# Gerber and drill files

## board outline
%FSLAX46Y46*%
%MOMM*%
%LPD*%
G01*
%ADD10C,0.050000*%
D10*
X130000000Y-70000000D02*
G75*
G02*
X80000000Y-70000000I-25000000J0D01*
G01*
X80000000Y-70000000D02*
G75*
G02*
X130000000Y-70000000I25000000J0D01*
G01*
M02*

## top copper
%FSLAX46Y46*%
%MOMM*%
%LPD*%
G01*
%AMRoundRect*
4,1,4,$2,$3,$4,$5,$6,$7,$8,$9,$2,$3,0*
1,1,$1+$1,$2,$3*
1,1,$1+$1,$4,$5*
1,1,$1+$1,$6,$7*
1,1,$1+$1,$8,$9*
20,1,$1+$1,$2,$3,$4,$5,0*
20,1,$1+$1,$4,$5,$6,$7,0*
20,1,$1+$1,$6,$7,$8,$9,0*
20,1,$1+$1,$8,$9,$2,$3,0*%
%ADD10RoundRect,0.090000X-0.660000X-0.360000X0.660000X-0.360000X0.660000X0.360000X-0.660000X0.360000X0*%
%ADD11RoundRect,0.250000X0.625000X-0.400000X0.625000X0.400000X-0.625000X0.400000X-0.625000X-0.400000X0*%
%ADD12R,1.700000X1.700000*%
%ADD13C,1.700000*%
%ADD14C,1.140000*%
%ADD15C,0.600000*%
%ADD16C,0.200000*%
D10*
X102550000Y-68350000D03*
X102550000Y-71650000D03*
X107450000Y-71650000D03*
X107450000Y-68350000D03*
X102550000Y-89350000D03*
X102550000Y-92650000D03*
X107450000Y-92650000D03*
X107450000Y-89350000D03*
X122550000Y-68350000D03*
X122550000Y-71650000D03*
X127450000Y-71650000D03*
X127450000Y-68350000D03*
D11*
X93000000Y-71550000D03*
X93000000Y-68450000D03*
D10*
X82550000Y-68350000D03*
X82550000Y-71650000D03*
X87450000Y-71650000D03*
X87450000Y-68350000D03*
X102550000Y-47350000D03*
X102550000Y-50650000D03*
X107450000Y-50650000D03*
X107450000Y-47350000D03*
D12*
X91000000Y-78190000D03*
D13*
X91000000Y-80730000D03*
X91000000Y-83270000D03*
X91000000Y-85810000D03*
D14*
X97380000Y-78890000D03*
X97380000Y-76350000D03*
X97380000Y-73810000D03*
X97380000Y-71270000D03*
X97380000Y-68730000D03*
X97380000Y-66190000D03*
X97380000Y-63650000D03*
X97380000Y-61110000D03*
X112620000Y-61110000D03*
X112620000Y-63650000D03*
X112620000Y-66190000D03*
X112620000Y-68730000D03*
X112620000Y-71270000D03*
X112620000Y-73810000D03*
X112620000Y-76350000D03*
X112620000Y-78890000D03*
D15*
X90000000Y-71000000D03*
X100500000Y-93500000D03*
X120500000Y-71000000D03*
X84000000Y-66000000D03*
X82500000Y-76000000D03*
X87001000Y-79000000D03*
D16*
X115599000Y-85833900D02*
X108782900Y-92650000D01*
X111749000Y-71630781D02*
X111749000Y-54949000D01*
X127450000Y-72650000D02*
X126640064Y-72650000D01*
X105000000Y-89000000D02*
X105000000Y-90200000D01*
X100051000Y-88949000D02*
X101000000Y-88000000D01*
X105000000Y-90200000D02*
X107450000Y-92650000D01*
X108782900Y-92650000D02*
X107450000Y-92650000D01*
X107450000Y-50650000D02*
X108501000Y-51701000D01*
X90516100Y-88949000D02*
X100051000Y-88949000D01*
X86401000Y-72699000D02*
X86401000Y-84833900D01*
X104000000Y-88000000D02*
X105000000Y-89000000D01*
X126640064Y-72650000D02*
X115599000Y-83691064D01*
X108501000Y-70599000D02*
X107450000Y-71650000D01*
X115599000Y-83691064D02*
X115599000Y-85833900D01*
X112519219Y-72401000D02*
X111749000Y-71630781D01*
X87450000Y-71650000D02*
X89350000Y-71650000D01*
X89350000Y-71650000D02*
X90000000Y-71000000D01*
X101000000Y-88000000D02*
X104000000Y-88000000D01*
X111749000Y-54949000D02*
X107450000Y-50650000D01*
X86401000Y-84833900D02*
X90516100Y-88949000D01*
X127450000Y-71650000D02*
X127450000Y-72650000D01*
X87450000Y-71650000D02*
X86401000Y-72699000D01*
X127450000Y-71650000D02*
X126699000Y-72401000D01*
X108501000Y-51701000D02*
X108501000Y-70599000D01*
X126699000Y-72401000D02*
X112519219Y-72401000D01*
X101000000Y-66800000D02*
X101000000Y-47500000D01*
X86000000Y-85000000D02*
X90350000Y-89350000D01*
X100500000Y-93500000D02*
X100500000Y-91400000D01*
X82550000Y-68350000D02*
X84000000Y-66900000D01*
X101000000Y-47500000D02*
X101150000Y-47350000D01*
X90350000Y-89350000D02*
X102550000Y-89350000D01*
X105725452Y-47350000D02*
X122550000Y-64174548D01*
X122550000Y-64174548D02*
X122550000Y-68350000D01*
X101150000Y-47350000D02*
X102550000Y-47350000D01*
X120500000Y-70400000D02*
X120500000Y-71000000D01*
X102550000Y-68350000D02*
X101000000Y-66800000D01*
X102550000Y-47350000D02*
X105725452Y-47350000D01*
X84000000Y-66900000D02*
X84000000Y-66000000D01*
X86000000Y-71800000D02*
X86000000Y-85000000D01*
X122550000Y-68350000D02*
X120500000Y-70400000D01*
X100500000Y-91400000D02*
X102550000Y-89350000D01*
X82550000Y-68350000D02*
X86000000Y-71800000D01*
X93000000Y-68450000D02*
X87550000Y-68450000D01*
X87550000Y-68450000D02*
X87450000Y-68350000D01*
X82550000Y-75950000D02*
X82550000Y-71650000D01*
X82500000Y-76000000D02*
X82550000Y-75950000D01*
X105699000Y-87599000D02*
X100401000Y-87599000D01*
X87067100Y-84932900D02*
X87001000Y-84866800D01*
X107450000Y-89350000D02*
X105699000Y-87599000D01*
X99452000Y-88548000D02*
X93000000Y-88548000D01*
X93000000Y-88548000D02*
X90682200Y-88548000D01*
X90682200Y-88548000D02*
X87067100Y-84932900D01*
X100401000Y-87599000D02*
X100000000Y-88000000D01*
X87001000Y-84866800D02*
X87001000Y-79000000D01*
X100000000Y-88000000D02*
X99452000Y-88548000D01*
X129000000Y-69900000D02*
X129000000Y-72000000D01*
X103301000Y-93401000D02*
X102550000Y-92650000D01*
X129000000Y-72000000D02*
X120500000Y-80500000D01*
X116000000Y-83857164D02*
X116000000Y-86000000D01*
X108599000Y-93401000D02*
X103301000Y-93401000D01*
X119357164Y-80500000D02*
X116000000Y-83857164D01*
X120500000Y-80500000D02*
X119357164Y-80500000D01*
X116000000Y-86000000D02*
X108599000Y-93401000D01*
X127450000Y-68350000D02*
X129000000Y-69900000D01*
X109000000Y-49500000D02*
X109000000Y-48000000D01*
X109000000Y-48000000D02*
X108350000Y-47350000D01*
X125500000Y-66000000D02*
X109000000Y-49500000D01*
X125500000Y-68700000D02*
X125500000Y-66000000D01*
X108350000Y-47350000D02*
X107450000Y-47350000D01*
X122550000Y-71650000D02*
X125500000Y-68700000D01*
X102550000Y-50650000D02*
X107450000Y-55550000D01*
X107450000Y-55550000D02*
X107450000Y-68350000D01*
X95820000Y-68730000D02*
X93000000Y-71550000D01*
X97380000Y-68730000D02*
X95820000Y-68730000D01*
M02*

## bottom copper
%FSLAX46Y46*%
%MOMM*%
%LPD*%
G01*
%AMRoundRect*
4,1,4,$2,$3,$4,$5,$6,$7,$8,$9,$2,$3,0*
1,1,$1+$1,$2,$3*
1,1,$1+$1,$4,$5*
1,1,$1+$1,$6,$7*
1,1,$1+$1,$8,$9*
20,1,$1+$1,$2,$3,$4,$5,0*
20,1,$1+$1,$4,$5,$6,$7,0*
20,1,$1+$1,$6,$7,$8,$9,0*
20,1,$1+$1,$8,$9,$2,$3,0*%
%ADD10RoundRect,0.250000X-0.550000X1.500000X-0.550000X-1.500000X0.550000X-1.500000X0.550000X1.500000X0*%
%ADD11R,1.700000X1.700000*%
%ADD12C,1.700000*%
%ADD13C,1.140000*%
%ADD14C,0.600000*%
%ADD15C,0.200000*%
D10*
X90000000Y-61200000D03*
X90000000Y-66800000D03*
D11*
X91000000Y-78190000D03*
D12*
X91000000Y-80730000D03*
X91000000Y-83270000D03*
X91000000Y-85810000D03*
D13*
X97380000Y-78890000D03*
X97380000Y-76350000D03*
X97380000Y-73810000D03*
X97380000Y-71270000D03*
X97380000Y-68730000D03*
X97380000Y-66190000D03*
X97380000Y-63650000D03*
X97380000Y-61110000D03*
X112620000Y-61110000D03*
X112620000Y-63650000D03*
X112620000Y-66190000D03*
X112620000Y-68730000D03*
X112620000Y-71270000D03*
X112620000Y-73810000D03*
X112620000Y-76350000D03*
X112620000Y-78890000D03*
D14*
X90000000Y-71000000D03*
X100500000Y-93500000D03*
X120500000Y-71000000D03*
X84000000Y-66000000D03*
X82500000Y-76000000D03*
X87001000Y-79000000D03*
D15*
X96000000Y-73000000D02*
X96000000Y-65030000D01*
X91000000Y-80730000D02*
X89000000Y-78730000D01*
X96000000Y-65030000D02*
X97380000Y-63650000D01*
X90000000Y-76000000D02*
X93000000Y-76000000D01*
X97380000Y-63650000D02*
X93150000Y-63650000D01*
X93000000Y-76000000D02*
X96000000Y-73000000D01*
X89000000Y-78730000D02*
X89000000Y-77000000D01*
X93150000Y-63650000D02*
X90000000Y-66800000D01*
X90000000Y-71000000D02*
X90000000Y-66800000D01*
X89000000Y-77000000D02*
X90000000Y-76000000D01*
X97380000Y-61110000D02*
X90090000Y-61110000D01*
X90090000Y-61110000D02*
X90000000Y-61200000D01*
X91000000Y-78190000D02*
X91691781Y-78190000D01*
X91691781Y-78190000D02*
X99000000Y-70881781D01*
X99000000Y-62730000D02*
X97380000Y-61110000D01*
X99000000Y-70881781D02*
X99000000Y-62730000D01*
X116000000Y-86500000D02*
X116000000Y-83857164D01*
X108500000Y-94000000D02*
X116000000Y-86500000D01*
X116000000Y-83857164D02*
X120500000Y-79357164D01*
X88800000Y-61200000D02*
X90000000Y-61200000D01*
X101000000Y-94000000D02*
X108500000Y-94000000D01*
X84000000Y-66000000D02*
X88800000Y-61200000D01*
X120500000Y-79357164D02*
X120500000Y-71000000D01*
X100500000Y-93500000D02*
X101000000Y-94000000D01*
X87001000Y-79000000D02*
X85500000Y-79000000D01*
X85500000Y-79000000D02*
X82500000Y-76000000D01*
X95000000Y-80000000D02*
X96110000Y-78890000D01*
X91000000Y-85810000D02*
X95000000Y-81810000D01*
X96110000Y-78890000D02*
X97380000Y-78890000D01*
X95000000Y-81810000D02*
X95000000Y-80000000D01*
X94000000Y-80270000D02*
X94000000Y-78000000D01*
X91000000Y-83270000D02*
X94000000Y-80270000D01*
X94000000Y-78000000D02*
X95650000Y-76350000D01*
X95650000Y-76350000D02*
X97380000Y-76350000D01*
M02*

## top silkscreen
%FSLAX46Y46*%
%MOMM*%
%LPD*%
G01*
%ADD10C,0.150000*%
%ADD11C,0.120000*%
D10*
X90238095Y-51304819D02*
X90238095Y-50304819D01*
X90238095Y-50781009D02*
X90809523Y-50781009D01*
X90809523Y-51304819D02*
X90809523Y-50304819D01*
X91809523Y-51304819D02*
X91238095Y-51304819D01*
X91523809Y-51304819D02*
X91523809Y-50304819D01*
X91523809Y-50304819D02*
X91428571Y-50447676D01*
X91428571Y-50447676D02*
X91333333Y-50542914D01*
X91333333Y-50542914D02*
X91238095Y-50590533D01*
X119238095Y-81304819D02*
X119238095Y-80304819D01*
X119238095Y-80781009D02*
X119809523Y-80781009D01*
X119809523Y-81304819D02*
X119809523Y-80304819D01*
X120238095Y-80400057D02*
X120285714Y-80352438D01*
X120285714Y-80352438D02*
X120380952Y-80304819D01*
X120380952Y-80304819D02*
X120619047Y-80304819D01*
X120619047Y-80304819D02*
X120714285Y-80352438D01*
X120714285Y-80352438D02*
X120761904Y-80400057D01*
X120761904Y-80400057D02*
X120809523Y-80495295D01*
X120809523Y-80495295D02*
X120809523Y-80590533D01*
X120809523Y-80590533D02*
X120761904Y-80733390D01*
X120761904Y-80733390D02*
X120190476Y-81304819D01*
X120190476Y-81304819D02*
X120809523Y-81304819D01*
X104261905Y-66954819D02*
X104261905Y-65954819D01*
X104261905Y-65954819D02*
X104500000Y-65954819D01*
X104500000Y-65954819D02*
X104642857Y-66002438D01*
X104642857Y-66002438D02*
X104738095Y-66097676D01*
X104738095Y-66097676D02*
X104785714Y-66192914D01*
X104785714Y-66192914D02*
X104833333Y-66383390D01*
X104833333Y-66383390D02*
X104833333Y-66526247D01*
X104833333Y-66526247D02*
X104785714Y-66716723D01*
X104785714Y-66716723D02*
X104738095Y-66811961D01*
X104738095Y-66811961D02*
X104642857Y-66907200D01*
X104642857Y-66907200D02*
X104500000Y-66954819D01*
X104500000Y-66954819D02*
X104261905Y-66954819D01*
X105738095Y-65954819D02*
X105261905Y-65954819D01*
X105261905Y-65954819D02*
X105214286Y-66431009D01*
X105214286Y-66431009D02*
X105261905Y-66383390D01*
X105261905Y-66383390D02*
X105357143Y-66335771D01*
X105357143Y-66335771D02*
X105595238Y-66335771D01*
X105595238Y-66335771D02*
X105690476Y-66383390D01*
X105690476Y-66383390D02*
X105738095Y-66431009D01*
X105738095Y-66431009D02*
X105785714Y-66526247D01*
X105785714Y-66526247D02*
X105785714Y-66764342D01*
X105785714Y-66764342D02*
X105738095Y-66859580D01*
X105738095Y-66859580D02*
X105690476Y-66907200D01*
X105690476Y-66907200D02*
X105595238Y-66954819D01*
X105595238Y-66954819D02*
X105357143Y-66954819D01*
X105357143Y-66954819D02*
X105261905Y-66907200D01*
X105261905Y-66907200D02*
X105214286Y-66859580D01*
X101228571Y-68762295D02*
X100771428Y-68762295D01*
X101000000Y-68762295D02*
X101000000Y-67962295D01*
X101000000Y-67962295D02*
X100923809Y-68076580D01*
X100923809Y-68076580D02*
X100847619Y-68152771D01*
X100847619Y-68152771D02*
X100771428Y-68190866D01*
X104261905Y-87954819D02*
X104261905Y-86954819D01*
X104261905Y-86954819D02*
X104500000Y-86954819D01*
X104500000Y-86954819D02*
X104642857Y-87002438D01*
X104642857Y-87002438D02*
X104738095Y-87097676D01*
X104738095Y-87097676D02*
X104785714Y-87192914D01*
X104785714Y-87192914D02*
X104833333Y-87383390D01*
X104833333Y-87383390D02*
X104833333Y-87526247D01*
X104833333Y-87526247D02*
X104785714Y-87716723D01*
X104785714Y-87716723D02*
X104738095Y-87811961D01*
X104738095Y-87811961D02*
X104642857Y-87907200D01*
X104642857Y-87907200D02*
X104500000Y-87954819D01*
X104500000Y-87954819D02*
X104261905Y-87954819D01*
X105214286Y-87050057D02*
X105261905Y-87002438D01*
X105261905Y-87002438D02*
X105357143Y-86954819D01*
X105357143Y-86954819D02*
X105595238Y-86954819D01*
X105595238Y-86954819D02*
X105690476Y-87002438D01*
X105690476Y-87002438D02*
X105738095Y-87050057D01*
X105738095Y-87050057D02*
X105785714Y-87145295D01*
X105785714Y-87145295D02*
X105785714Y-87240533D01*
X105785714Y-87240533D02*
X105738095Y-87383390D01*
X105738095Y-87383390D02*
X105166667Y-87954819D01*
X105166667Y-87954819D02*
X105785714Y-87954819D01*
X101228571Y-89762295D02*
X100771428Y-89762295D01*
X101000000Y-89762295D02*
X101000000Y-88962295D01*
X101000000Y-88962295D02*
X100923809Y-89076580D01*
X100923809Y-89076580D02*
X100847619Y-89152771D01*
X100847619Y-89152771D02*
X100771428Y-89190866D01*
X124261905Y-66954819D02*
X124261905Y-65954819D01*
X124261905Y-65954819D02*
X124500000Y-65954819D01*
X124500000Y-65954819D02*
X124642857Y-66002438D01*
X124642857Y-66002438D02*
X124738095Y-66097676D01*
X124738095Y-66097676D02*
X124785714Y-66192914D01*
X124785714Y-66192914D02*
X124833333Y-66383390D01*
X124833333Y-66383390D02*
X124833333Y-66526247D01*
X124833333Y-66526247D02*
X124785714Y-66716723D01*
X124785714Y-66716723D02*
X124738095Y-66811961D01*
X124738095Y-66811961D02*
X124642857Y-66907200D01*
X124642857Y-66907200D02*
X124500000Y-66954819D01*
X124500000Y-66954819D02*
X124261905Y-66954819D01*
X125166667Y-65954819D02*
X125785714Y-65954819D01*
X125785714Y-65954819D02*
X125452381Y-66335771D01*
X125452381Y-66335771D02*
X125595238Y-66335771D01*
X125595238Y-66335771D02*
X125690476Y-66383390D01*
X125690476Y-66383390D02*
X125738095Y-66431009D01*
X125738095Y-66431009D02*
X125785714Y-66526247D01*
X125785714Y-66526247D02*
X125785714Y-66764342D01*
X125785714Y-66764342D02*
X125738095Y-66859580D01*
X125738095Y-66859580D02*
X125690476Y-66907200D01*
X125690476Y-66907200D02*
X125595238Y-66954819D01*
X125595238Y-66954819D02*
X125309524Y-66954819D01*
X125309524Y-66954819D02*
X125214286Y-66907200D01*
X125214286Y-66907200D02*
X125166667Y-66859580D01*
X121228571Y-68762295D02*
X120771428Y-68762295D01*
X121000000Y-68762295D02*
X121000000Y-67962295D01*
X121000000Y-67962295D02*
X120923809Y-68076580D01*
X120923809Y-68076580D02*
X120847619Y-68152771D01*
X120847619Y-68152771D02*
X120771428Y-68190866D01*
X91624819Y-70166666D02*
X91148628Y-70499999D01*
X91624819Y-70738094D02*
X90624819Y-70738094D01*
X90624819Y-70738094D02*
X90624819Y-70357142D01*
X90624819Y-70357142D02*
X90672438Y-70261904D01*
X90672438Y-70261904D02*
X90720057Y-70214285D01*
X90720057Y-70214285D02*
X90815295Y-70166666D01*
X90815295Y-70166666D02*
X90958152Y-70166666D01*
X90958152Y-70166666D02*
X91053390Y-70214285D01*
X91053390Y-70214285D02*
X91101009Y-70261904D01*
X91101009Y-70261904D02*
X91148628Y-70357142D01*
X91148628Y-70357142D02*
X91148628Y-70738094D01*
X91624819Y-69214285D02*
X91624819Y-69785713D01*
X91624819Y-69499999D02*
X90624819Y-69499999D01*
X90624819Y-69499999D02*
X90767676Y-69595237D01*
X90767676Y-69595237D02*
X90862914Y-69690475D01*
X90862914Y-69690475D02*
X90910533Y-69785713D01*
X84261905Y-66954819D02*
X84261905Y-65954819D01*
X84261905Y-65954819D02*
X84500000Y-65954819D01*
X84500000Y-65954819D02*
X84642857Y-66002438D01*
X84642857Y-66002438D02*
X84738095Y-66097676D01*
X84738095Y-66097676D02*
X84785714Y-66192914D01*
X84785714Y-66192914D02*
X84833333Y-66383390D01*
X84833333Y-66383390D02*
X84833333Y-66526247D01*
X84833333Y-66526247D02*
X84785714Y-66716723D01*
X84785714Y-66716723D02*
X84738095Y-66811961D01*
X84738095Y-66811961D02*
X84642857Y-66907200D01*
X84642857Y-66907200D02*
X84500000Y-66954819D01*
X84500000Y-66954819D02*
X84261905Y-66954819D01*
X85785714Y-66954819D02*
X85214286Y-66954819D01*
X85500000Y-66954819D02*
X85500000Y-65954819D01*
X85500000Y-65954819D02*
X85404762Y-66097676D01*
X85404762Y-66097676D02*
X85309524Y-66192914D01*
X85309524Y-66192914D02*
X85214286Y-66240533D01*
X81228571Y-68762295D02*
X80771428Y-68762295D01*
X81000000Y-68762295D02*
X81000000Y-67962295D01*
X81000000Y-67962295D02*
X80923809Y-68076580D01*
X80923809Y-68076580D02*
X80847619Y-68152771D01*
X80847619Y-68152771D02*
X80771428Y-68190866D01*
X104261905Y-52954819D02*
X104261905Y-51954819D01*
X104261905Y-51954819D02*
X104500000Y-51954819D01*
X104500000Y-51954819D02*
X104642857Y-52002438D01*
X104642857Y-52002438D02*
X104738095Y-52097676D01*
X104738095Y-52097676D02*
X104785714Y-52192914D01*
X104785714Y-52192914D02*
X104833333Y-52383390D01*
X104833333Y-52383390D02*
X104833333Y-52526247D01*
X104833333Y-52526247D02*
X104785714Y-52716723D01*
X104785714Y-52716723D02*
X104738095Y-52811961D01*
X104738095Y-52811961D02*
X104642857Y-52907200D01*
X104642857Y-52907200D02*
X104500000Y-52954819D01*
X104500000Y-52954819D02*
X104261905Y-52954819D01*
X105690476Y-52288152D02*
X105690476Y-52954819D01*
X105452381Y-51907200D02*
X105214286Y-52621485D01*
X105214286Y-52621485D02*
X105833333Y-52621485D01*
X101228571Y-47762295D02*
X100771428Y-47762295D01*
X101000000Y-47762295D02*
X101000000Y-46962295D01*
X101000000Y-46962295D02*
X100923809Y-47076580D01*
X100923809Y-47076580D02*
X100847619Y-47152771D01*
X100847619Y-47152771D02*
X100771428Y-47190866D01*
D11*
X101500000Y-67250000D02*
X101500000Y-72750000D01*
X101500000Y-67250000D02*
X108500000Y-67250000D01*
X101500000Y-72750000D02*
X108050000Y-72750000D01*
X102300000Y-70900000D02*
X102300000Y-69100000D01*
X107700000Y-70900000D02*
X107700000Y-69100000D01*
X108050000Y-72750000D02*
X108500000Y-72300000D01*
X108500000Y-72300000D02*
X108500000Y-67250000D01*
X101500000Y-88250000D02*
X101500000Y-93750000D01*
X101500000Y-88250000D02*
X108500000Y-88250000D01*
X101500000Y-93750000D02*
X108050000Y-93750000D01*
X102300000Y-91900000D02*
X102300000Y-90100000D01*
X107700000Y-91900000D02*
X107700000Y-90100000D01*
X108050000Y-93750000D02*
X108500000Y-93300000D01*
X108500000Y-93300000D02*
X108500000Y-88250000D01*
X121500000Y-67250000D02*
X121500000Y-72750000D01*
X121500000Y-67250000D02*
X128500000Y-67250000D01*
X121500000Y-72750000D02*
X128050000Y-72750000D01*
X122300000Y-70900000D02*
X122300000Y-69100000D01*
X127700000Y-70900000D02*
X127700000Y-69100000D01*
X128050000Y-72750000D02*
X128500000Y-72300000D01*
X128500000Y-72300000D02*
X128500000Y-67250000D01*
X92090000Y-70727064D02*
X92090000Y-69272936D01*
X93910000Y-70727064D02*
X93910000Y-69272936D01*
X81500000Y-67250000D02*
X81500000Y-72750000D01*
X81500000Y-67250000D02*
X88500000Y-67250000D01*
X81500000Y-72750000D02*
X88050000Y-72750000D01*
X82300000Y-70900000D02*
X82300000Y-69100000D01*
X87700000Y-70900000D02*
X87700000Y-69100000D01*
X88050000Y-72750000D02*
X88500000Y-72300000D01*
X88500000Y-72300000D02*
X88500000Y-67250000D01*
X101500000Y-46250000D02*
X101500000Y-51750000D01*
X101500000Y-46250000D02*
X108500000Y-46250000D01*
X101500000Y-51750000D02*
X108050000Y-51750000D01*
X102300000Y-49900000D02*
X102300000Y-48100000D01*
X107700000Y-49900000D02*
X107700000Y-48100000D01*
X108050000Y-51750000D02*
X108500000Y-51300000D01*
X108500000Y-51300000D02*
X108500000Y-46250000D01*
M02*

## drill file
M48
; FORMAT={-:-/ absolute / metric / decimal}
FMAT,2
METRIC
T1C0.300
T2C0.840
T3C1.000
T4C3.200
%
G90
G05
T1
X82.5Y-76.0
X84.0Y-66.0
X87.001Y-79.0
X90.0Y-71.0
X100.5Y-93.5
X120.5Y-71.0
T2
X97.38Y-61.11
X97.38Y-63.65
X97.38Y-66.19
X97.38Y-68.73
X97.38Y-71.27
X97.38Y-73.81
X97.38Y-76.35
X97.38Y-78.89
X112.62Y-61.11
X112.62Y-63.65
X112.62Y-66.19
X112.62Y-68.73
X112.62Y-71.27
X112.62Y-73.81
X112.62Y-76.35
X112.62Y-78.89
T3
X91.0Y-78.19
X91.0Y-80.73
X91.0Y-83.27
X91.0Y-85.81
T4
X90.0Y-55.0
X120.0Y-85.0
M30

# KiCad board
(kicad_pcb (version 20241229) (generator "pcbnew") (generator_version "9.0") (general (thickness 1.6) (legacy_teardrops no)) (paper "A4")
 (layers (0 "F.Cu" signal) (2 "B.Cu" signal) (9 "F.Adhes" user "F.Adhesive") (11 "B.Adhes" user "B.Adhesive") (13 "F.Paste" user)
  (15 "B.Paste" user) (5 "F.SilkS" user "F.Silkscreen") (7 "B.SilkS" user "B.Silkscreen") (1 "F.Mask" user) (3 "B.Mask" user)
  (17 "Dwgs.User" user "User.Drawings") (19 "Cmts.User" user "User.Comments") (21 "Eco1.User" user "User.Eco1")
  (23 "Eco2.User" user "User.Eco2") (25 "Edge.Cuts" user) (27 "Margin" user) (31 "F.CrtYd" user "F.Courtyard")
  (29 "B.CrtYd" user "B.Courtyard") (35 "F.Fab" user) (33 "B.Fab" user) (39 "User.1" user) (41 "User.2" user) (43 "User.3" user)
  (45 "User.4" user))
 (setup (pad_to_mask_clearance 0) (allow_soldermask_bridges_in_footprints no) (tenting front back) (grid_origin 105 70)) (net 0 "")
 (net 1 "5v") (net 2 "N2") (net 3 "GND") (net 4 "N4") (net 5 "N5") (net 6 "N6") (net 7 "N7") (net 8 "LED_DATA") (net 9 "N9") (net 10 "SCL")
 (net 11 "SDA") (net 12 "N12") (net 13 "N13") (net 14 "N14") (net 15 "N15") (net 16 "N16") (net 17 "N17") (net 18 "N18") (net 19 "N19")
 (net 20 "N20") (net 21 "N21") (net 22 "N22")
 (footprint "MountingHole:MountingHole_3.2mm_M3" (layer "F.Cu") (at 90 55)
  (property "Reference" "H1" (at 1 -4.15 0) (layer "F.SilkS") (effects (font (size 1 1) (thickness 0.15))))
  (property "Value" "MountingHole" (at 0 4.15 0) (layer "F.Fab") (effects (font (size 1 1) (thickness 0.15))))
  (pad "" np_thru_hole circle (at 0 0) (size 3.2 3.2) (drill 3.2) (layers "*.Cu" "*.Mask")))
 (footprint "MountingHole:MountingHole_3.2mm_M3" (layer "F.Cu") (at 120 85)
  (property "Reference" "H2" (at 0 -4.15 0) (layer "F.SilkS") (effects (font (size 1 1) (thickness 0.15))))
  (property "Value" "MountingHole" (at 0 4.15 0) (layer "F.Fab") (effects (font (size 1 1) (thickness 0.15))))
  (pad "" np_thru_hole circle (at 0 0) (size 3.2 3.2) (drill 3.2) (layers "*.Cu" "*.Mask")))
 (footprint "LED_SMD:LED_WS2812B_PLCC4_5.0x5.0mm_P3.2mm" (layer "F.Cu") (at 105 70)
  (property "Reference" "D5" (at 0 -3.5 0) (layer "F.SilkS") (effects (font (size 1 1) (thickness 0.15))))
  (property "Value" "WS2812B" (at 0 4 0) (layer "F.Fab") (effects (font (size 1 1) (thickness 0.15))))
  (fp_line (start -3.5 -2.75) (end -3.5 2.75) (stroke (width 0.12) (type default)) (layer "F.SilkS"))
  (fp_line (start -3.5 -2.75) (end 3.5 -2.75) (stroke (width 0.12) (type solid)) (layer "F.SilkS"))
  (fp_line (start -3.5 2.75) (end 3.05 2.75) (stroke (width 0.12) (type solid)) (layer "F.SilkS"))
  (fp_line (start -2.7 0.9) (end -2.7 -0.9) (stroke (width 0.12) (type default)) (layer "F.SilkS"))
  (fp_line (start 2.7 0.9) (end 2.7 -0.9) (stroke (width 0.12) (type default)) (layer "F.SilkS"))
  (fp_line (start 3.05 2.75) (end 3.5 2.3) (stroke (width 0.12) (type default)) (layer "F.SilkS"))
  (fp_line (start 3.5 2.3) (end 3.5 -2.75) (stroke (width 0.12) (type default)) (layer "F.SilkS"))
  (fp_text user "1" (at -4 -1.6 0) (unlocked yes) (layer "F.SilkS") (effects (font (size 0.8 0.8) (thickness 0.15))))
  (pad "1" smd roundrect (at -2.45 -1.65) (size 1.5 0.9) (layers "F.Cu" "F.Mask" "F.Paste") (roundrect_rratio 0.1) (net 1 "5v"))
  (pad "2" smd roundrect (at -2.45 1.65) (size 1.5 0.9) (layers "F.Cu" "F.Mask" "F.Paste") (roundrect_rratio 0.1) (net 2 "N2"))
  (pad "3" smd roundrect (at 2.45 1.65) (size 1.5 0.9) (layers "F.Cu" "F.Mask" "F.Paste") (roundrect_rratio 0.1) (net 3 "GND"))
  (pad "4" smd roundrect (at 2.45 -1.65) (size 1.5 0.9) (layers "F.Cu" "F.Mask" "F.Paste") (roundrect_rratio 0.1) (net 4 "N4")))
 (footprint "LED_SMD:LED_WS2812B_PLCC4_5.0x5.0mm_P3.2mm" (layer "F.Cu") (at 105 91)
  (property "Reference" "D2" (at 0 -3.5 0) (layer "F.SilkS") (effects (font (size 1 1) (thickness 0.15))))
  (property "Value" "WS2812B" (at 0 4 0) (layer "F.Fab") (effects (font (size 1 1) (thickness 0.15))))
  (fp_line (start -3.5 -2.75) (end -3.5 2.75) (stroke (width 0.12) (type default)) (layer "F.SilkS"))
  (fp_line (start -3.5 -2.75) (end 3.5 -2.75) (stroke (width 0.12) (type solid)) (layer "F.SilkS"))
  (fp_line (start -3.5 2.75) (end 3.05 2.75) (stroke (width 0.12) (type solid)) (layer "F.SilkS"))
  (fp_line (start -2.7 0.9) (end -2.7 -0.9) (stroke (width 0.12) (type default)) (layer "F.SilkS"))
  (fp_line (start 2.7 0.9) (end 2.7 -0.9) (stroke (width 0.12) (type default)) (layer "F.SilkS"))
  (fp_line (start 3.05 2.75) (end 3.5 2.3) (stroke (width 0.12) (type default)) (layer "F.SilkS"))
  (fp_line (start 3.5 2.3) (end 3.5 -2.75) (stroke (width 0.12) (type default)) (layer "F.SilkS"))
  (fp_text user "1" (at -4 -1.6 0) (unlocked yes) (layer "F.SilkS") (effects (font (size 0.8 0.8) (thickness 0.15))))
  (pad "1" smd roundrect (at -2.45 -1.65) (size 1.5 0.9) (layers "F.Cu" "F.Mask" "F.Paste") (roundrect_rratio 0.1) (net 1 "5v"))
  (pad "2" smd roundrect (at -2.45 1.65) (size 1.5 0.9) (layers "F.Cu" "F.Mask" "F.Paste") (roundrect_rratio 0.1) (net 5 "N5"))
  (pad "3" smd roundrect (at 2.45 1.65) (size 1.5 0.9) (layers "F.Cu" "F.Mask" "F.Paste") (roundrect_rratio 0.1) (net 3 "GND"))
  (pad "4" smd roundrect (at 2.45 -1.65) (size 1.5 0.9) (layers "F.Cu" "F.Mask" "F.Paste") (roundrect_rratio 0.1) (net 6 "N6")))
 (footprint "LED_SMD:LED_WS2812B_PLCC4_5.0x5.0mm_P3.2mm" (layer "F.Cu") (at 125 70)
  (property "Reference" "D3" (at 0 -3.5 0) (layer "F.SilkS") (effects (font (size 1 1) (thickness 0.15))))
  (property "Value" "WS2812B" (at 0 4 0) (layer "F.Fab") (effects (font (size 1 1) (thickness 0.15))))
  (fp_line (start -3.5 -2.75) (end -3.5 2.75) (stroke (width 0.12) (type default)) (layer "F.SilkS"))
  (fp_line (start -3.5 -2.75) (end 3.5 -2.75) (stroke (width 0.12) (type solid)) (layer "F.SilkS"))
  (fp_line (start -3.5 2.75) (end 3.05 2.75) (stroke (width 0.12) (type solid)) (layer "F.SilkS"))
  (fp_line (start -2.7 0.9) (end -2.7 -0.9) (stroke (width 0.12) (type default)) (layer "F.SilkS"))
  (fp_line (start 2.7 0.9) (end 2.7 -0.9) (stroke (width 0.12) (type default)) (layer "F.SilkS"))
  (fp_line (start 3.05 2.75) (end 3.5 2.3) (stroke (width 0.12) (type default)) (layer "F.SilkS"))
  (fp_line (start 3.5 2.3) (end 3.5 -2.75) (stroke (width 0.12) (type default)) (layer "F.SilkS"))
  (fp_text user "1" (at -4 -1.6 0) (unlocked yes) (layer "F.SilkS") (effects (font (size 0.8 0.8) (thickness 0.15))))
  (pad "1" smd roundrect (at -2.45 -1.65) (size 1.5 0.9) (layers "F.Cu" "F.Mask" "F.Paste") (roundrect_rratio 0.1) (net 1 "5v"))
  (pad "2" smd roundrect (at -2.45 1.65) (size 1.5 0.9) (layers "F.Cu" "F.Mask" "F.Paste") (roundrect_rratio 0.1) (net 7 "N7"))
  (pad "3" smd roundrect (at 2.45 1.65) (size 1.5 0.9) (layers "F.Cu" "F.Mask" "F.Paste") (roundrect_rratio 0.1) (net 3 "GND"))
  (pad "4" smd roundrect (at 2.45 -1.65) (size 1.5 0.9) (layers "F.Cu" "F.Mask" "F.Paste") (roundrect_rratio 0.1) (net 5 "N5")))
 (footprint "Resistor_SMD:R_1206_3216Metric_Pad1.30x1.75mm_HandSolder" (layer "F.Cu") (at 93 70 90)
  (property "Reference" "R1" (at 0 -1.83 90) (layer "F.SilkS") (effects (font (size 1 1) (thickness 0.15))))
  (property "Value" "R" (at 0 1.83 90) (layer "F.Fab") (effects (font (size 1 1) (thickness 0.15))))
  (fp_line (start -0.727064 -0.91) (end 0.727064 -0.91) (stroke (width 0.12) (type solid)) (layer "F.SilkS"))
  (fp_line (start -0.727064 0.91) (end 0.727064 0.91) (stroke (width 0.12) (type solid)) (layer "F.SilkS"))
  (pad "1" smd roundrect (at -1.55 0 90) (size 1.3 1.75) (layers "F.Cu" "F.Mask" "F.Paste") (roundrect_rratio 0.192308) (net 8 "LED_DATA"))
  (pad "2" smd roundrect (at 1.55 0 90) (size 1.3 1.75) (layers "F.Cu" "F.Mask" "F.Paste") (roundrect_rratio 0.192308) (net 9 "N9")))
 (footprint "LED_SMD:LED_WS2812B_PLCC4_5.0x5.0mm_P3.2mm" (layer "F.Cu") (at 85 70)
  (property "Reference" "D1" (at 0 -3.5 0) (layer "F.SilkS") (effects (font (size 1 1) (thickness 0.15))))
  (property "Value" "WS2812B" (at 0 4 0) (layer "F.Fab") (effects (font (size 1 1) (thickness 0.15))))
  (fp_line (start -3.5 -2.75) (end -3.5 2.75) (stroke (width 0.12) (type default)) (layer "F.SilkS"))
  (fp_line (start -3.5 -2.75) (end 3.5 -2.75) (stroke (width 0.12) (type solid)) (layer "F.SilkS"))
  (fp_line (start -3.5 2.75) (end 3.05 2.75) (stroke (width 0.12) (type solid)) (layer "F.SilkS"))
  (fp_line (start -2.7 0.9) (end -2.7 -0.9) (stroke (width 0.12) (type default)) (layer "F.SilkS"))
  (fp_line (start 2.7 0.9) (end 2.7 -0.9) (stroke (width 0.12) (type default)) (layer "F.SilkS"))
  (fp_line (start 3.05 2.75) (end 3.5 2.3) (stroke (width 0.12) (type default)) (layer "F.SilkS"))
  (fp_line (start 3.5 2.3) (end 3.5 -2.75) (stroke (width 0.12) (type default)) (layer "F.SilkS"))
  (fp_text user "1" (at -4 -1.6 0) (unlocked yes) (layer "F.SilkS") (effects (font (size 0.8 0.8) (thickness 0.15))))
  (pad "1" smd roundrect (at -2.45 -1.65) (size 1.5 0.9) (layers "F.Cu" "F.Mask" "F.Paste") (roundrect_rratio 0.1) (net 1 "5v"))
  (pad "2" smd roundrect (at -2.45 1.65) (size 1.5 0.9) (layers "F.Cu" "F.Mask" "F.Paste") (roundrect_rratio 0.1) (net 6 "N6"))
  (pad "3" smd roundrect (at 2.45 1.65) (size 1.5 0.9) (layers "F.Cu" "F.Mask" "F.Paste") (roundrect_rratio 0.1) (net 3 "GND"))
  (pad "4" smd roundrect (at 2.45 -1.65) (size 1.5 0.9) (layers "F.Cu" "F.Mask" "F.Paste") (roundrect_rratio 0.1) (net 9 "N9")))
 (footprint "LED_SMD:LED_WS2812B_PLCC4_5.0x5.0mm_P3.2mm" (layer "F.Cu") (at 105 49)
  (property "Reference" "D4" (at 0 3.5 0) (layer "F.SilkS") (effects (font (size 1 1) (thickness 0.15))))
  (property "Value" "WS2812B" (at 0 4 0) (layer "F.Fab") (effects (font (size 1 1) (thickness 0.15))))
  (fp_line (start -3.5 -2.75) (end -3.5 2.75) (stroke (width 0.12) (type default)) (layer "F.SilkS"))
  (fp_line (start -3.5 -2.75) (end 3.5 -2.75) (stroke (width 0.12) (type solid)) (layer "F.SilkS"))
  (fp_line (start -3.5 2.75) (end 3.05 2.75) (stroke (width 0.12) (type solid)) (layer "F.SilkS"))
  (fp_line (start -2.7 0.9) (end -2.7 -0.9) (stroke (width 0.12) (type default)) (layer "F.SilkS"))
  (fp_line (start 2.7 0.9) (end 2.7 -0.9) (stroke (width 0.12) (type default)) (layer "F.SilkS"))
  (fp_line (start 3.05 2.75) (end 3.5 2.3) (stroke (width 0.12) (type default)) (layer "F.SilkS"))
  (fp_line (start 3.5 2.3) (end 3.5 -2.75) (stroke (width 0.12) (type default)) (layer "F.SilkS"))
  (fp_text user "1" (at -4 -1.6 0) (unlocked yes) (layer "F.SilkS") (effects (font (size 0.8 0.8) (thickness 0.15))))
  (pad "1" smd roundrect (at -2.45 -1.65) (size 1.5 0.9) (layers "F.Cu" "F.Mask" "F.Paste") (roundrect_rratio 0.1) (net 1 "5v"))
  (pad "2" smd roundrect (at -2.45 1.65) (size 1.5 0.9) (layers "F.Cu" "F.Mask" "F.Paste") (roundrect_rratio 0.1) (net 4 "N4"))
  (pad "3" smd roundrect (at 2.45 1.65) (size 1.5 0.9) (layers "F.Cu" "F.Mask" "F.Paste") (roundrect_rratio 0.1) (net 3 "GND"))
  (pad "4" smd roundrect (at 2.45 -1.65) (size 1.5 0.9) (layers "F.Cu" "F.Mask" "F.Paste") (roundrect_rratio 0.1) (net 7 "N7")))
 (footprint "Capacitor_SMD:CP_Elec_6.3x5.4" (layer "B.Cu") (at 90 64 -90)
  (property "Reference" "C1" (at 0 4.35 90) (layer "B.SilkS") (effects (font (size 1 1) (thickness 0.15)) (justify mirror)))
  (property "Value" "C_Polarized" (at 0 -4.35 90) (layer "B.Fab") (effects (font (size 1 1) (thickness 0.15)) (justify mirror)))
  (pad "1" smd roundrect (at -2.8 0 270) (size 3.5 1.6) (layers "B.Cu" "B.Mask" "B.Paste") (roundrect_rratio 0.15625) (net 1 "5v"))
  (pad "2" smd roundrect (at 2.8 0 270) (size 3.5 1.6) (layers "B.Cu" "B.Mask" "B.Paste") (roundrect_rratio 0.15625) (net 3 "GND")))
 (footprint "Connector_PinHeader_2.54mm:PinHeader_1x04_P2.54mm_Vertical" (layer "B.Cu") (at 91 78.19 180)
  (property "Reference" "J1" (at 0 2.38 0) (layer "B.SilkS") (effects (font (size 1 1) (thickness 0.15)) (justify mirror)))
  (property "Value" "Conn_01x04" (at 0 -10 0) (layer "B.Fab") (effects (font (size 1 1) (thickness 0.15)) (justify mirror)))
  (pad "1" thru_hole rect (at 0 0 180) (size 1.7 1.7) (drill 1) (layers "*.Cu" "*.Mask") (remove_unused_layers no) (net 1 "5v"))
  (pad "2" thru_hole circle (at 0 -2.54 180) (size 1.7 1.7) (drill 1) (layers "*.Cu" "*.Mask") (remove_unused_layers no) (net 3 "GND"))
  (pad "3" thru_hole circle (at 0 -5.08 180) (size 1.7 1.7) (drill 1) (layers "*.Cu" "*.Mask") (remove_unused_layers no) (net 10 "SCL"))
  (pad "4" thru_hole circle (at 0 -7.62 180) (size 1.7 1.7) (drill 1) (layers "*.Cu" "*.Mask") (remove_unused_layers no) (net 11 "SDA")))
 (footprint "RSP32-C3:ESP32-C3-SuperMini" (layer "B.Cu") (at 105 70 180)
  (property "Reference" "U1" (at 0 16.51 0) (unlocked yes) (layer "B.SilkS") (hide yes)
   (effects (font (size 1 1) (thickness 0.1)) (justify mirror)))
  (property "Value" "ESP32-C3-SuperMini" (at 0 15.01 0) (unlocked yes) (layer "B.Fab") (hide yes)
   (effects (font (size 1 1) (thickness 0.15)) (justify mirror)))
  (pad "1" thru_hole circle (at 7.62 -8.89 180) (size 1.14 1.14) (drill 0.84) (layers "*.Cu" "*.Mask") (remove_unused_layers no)
   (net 11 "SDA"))
  (pad "2" thru_hole circle (at 7.62 -6.35 180) (size 1.14 1.14) (drill 0.84) (layers "*.Cu" "*.Mask") (remove_unused_layers no)
   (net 10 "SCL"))
  (pad "3" thru_hole circle (at 7.62 -3.81 180) (size 1.14 1.14) (drill 0.84) (layers "*.Cu" "*.Mask") (remove_unused_layers no)
   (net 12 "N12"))
  (pad "4" thru_hole circle (at 7.62 -1.27 180) (size 1.14 1.14) (drill 0.84) (layers "*.Cu" "*.Mask") (remove_unused_layers no)
   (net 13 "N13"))
  (pad "5" thru_hole circle (at 7.62 1.27 180) (size 1.14 1.14) (drill 0.84) (layers "*.Cu" "*.Mask") (remove_unused_layers no)
   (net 8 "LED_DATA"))
  (pad "6" thru_hole circle (at 7.62 3.81 180) (size 1.14 1.14) (drill 0.84) (layers "*.Cu" "*.Mask") (remove_unused_layers no)
   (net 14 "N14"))
  (pad "7" thru_hole circle (at 7.62 6.35 180) (size 1.14 1.14) (drill 0.84) (layers "*.Cu" "*.Mask") (remove_unused_layers no)
   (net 3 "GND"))
  (pad "8" thru_hole circle (at 7.62 8.89 180) (size 1.14 1.14) (drill 0.84) (layers "*.Cu" "*.Mask") (remove_unused_layers no) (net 1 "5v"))
  (pad "9" thru_hole circle (at -7.62 8.89 180) (size 1.14 1.14) (drill 0.84) (layers "*.Cu" "*.Mask") (remove_unused_layers no)
   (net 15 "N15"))
  (pad "10" thru_hole circle (at -7.62 6.35 180) (size 1.14 1.14) (drill 0.84) (layers "*.Cu" "*.Mask") (remove_unused_layers no)
   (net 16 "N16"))
  (pad "11" thru_hole circle (at -7.62 3.81 180) (size 1.14 1.14) (drill 0.84) (layers "*.Cu" "*.Mask") (remove_unused_layers no)
   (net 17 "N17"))
  (pad "12" thru_hole circle (at -7.62 1.27 180) (size 1.14 1.14) (drill 0.84) (layers "*.Cu" "*.Mask") (remove_unused_layers no)
   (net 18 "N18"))
  (pad "13" thru_hole circle (at -7.62 -1.27 180) (size 1.14 1.14) (drill 0.84) (layers "*.Cu" "*.Mask") (remove_unused_layers no)
   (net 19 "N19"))
  (pad "14" thru_hole circle (at -7.62 -3.81 180) (size 1.14 1.14) (drill 0.84) (layers "*.Cu" "*.Mask") (remove_unused_layers no)
   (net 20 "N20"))
  (pad "15" thru_hole circle (at -7.62 -6.35 180) (size 1.14 1.14) (drill 0.84) (layers "*.Cu" "*.Mask") (remove_unused_layers no)
   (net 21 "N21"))
  (pad "16" thru_hole circle (at -7.62 -8.89 180) (size 1.14 1.14) (drill 0.84) (layers "*.Cu" "*.Mask") (remove_unused_layers no)
   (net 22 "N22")))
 (gr_circle (center 105 70) (end 130 70) (stroke (width 0.05) (type default)) (fill no) (layer "Edge.Cuts"))
 (segment (start 115.599 85.8339) (end 108.7829 92.65) (width 0.2) (layer "F.Cu") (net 3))
 (segment (start 111.749 71.630781) (end 111.749 54.949) (width 0.2) (layer "F.Cu") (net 3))
 (segment (start 127.45 72.65) (end 126.640064 72.65) (width 0.2) (layer "F.Cu") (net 3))
 (segment (start 105 89) (end 105 90.2) (width 0.2) (layer "F.Cu") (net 3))
 (segment (start 100.051 88.949) (end 101 88) (width 0.2) (layer "F.Cu") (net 3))
 (segment (start 105 90.2) (end 107.45 92.65) (width 0.2) (layer "F.Cu") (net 3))
 (segment (start 108.7829 92.65) (end 107.45 92.65) (width 0.2) (layer "F.Cu") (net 3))
 (segment (start 107.45 50.65) (end 108.501 51.701) (width 0.2) (layer "F.Cu") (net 3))
 (segment (start 90.5161 88.949) (end 100.051 88.949) (width 0.2) (layer "F.Cu") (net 3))
 (segment (start 86.401 72.699) (end 86.401 84.8339) (width 0.2) (layer "F.Cu") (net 3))
 (segment (start 104 88) (end 105 89) (width 0.2) (layer "F.Cu") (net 3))
 (segment (start 126.640064 72.65) (end 115.599 83.691064) (width 0.2) (layer "F.Cu") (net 3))
 (segment (start 108.501 70.599) (end 107.45 71.65) (width 0.2) (layer "F.Cu") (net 3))
 (segment (start 115.599 83.691064) (end 115.599 85.8339) (width 0.2) (layer "F.Cu") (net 3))
 (segment (start 112.519219 72.401) (end 111.749 71.630781) (width 0.2) (layer "F.Cu") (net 3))
 (segment (start 87.45 71.65) (end 89.35 71.65) (width 0.2) (layer "F.Cu") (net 3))
 (segment (start 89.35 71.65) (end 90 71) (width 0.2) (layer "F.Cu") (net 3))
 (segment (start 101 88) (end 104 88) (width 0.2) (layer "F.Cu") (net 3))
 (segment (start 111.749 54.949) (end 107.45 50.65) (width 0.2) (layer "F.Cu") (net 3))
 (segment (start 86.401 84.8339) (end 90.5161 88.949) (width 0.2) (layer "F.Cu") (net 3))
 (segment (start 127.45 71.65) (end 127.45 72.65) (width 0.2) (layer "F.Cu") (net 3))
 (segment (start 87.45 71.65) (end 86.401 72.699) (width 0.2) (layer "F.Cu") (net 3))
 (segment (start 127.45 71.65) (end 126.699 72.401) (width 0.2) (layer "F.Cu") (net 3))
 (segment (start 108.501 51.701) (end 108.501 70.599) (width 0.2) (layer "F.Cu") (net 3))
 (segment (start 126.699 72.401) (end 112.519219 72.401) (width 0.2) (layer "F.Cu") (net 3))
 (via (at 90 71) (size 0.6) (drill 0.3) (layers "F.Cu" "B.Cu") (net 3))
 (segment (start 96 73) (end 96 65.03) (width 0.2) (layer "B.Cu") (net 3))
 (segment (start 91 80.73) (end 89 78.73) (width 0.2) (layer "B.Cu") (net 3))
 (segment (start 96 65.03) (end 97.38 63.65) (width 0.2) (layer "B.Cu") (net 3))
 (segment (start 90 76) (end 93 76) (width 0.2) (layer "B.Cu") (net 3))
 (segment (start 97.38 63.65) (end 93.15 63.65) (width 0.2) (layer "B.Cu") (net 3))
 (segment (start 93 76) (end 96 73) (width 0.2) (layer "B.Cu") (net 3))
 (segment (start 89 78.73) (end 89 77) (width 0.2) (layer "B.Cu") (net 3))
 (segment (start 93.15 63.65) (end 90 66.8) (width 0.2) (layer "B.Cu") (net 3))
 (segment (start 90 71) (end 90 66.8) (width 0.2) (layer "B.Cu") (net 3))
 (segment (start 89 77) (end 90 76) (width 0.2) (layer "B.Cu") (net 3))
 (segment (start 101 66.8) (end 101 47.5) (width 0.2) (layer "F.Cu") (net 1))
 (segment (start 86 85) (end 90.35 89.35) (width 0.2) (layer "F.Cu") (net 1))
 (segment (start 100.5 93.5) (end 100.5 91.4) (width 0.2) (layer "F.Cu") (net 1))
 (segment (start 82.55 68.35) (end 84 66.9) (width 0.2) (layer "F.Cu") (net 1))
 (segment (start 101 47.5) (end 101.15 47.35) (width 0.2) (layer "F.Cu") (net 1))
 (segment (start 90.35 89.35) (end 102.55 89.35) (width 0.2) (layer "F.Cu") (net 1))
 (segment (start 105.725452 47.35) (end 122.55 64.174548) (width 0.2) (layer "F.Cu") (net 1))
 (segment (start 122.55 64.174548) (end 122.55 68.35) (width 0.2) (layer "F.Cu") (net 1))
 (segment (start 101.15 47.35) (end 102.55 47.35) (width 0.2) (layer "F.Cu") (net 1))
 (segment (start 120.5 70.4) (end 120.5 71) (width 0.2) (layer "F.Cu") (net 1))
 (segment (start 102.55 68.35) (end 101 66.8) (width 0.2) (layer "F.Cu") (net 1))
 (segment (start 102.55 47.35) (end 105.725452 47.35) (width 0.2) (layer "F.Cu") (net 1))
 (segment (start 84 66.9) (end 84 66) (width 0.2) (layer "F.Cu") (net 1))
 (segment (start 86 71.8) (end 86 85) (width 0.2) (layer "F.Cu") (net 1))
 (segment (start 122.55 68.35) (end 120.5 70.4) (width 0.2) (layer "F.Cu") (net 1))
 (segment (start 100.5 91.4) (end 102.55 89.35) (width 0.2) (layer "F.Cu") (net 1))
 (segment (start 82.55 68.35) (end 86 71.8) (width 0.2) (layer "F.Cu") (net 1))
 (via (at 100.5 93.5) (size 0.6) (drill 0.3) (layers "F.Cu" "B.Cu") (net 1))
 (via (at 120.5 71) (size 0.6) (drill 0.3) (layers "F.Cu" "B.Cu") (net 1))
 (via (at 84 66) (size 0.6) (drill 0.3) (layers "F.Cu" "B.Cu") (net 1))
 (segment (start 97.38 61.11) (end 90.09 61.11) (width 0.2) (layer "B.Cu") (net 1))
 (segment (start 90.09 61.11) (end 90 61.2) (width 0.2) (layer "B.Cu") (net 1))
 (segment (start 91 78.19) (end 91.691781 78.19) (width 0.2) (layer "B.Cu") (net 1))
 (segment (start 91.691781 78.19) (end 99 70.881781) (width 0.2) (layer "B.Cu") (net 1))
 (segment (start 99 62.73) (end 97.38 61.11) (width 0.2) (layer "B.Cu") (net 1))
 (segment (start 99 70.881781) (end 99 62.73) (width 0.2) (layer "B.Cu") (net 1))
 (segment (start 116 86.5) (end 116 83.857164) (width 0.2) (layer "B.Cu") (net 1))
 (segment (start 108.5 94) (end 116 86.5) (width 0.2) (layer "B.Cu") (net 1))
 (segment (start 116 83.857164) (end 120.5 79.357164) (width 0.2) (layer "B.Cu") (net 1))
 (segment (start 88.8 61.2) (end 90 61.2) (width 0.2) (layer "B.Cu") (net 1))
 (segment (start 101 94) (end 108.5 94) (width 0.2) (layer "B.Cu") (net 1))
 (segment (start 84 66) (end 88.8 61.2) (width 0.2) (layer "B.Cu") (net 1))
 (segment (start 120.5 79.357164) (end 120.5 71) (width 0.2) (layer "B.Cu") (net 1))
 (segment (start 100.5 93.5) (end 101 94) (width 0.2) (layer "B.Cu") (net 1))
 (segment (start 93 68.45) (end 87.55 68.45) (width 0.2) (layer "F.Cu") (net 9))
 (segment (start 87.55 68.45) (end 87.45 68.35) (width 0.2) (layer "F.Cu") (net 9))
 (segment (start 82.55 75.95) (end 82.55 71.65) (width 0.2) (layer "F.Cu") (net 6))
 (segment (start 82.5 76) (end 82.55 75.95) (width 0.2) (layer "F.Cu") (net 6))
 (segment (start 105.699 87.599) (end 100.401 87.599) (width 0.2) (layer "F.Cu") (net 6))
 (segment (start 87.0671 84.9329) (end 87.001 84.8668) (width 0.2) (layer "F.Cu") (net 6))
 (segment (start 107.45 89.35) (end 105.699 87.599) (width 0.2) (layer "F.Cu") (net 6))
 (segment (start 99.452 88.548) (end 93 88.548) (width 0.2) (layer "F.Cu") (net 6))
 (segment (start 93 88.548) (end 90.6822 88.548) (width 0.2) (layer "F.Cu") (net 6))
 (segment (start 90.6822 88.548) (end 87.0671 84.9329) (width 0.2) (layer "F.Cu") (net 6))
 (segment (start 100.401 87.599) (end 100 88) (width 0.2) (layer "F.Cu") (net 6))
 (segment (start 87.001 84.8668) (end 87.001 79) (width 0.2) (layer "F.Cu") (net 6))
 (segment (start 100 88) (end 99.452 88.548) (width 0.2) (layer "F.Cu") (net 6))
 (via (at 82.5 76) (size 0.6) (drill 0.3) (layers "F.Cu" "B.Cu") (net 6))
 (via (at 87.001 79) (size 0.6) (drill 0.3) (layers "F.Cu" "B.Cu") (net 6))
 (segment (start 87.001 79) (end 85.5 79) (width 0.2) (layer "B.Cu") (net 6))
 (segment (start 85.5 79) (end 82.5 76) (width 0.2) (layer "B.Cu") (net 6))
 (segment (start 129 69.9) (end 129 72) (width 0.2) (layer "F.Cu") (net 5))
 (segment (start 103.301 93.401) (end 102.55 92.65) (width 0.2) (layer "F.Cu") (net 5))
 (segment (start 129 72) (end 120.5 80.5) (width 0.2) (layer "F.Cu") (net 5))
 (segment (start 116 83.857164) (end 116 86) (width 0.2) (layer "F.Cu") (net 5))
 (segment (start 108.599 93.401) (end 103.301 93.401) (width 0.2) (layer "F.Cu") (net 5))
 (segment (start 119.357164 80.5) (end 116 83.857164) (width 0.2) (layer "F.Cu") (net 5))
 (segment (start 120.5 80.5) (end 119.357164 80.5) (width 0.2) (layer "F.Cu") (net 5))
 (segment (start 116 86) (end 108.599 93.401) (width 0.2) (layer "F.Cu") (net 5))
 (segment (start 127.45 68.35) (end 129 69.9) (width 0.2) (layer "F.Cu") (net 5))
 (segment (start 109 49.5) (end 109 48) (width 0.2) (layer "F.Cu") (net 7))
 (segment (start 109 48) (end 108.35 47.35) (width 0.2) (layer "F.Cu") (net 7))
 (segment (start 125.5 66) (end 109 49.5) (width 0.2) (layer "F.Cu") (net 7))
 (segment (start 125.5 68.7) (end 125.5 66) (width 0.2) (layer "F.Cu") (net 7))
 (segment (start 108.35 47.35) (end 107.45 47.35) (width 0.2) (layer "F.Cu") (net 7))
 (segment (start 122.55 71.65) (end 125.5 68.7) (width 0.2) (layer "F.Cu") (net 7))
 (segment (start 102.55 50.65) (end 107.45 55.55) (width 0.2) (layer "F.Cu") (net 4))
 (segment (start 107.45 55.55) (end 107.45 68.35) (width 0.2) (layer "F.Cu") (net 4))
 (segment (start 95 80) (end 96.11 78.89) (width 0.2) (layer "B.Cu") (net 11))
 (segment (start 91 85.81) (end 95 81.81) (width 0.2) (layer "B.Cu") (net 11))
 (segment (start 96.11 78.89) (end 97.38 78.89) (width 0.2) (layer "B.Cu") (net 11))
 (segment (start 95 81.81) (end 95 80) (width 0.2) (layer "B.Cu") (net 11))
 (segment (start 94 80.27) (end 94 78) (width 0.2) (layer "B.Cu") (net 10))
 (segment (start 91 83.27) (end 94 80.27) (width 0.2) (layer "B.Cu") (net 10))
 (segment (start 94 78) (end 95.65 76.35) (width 0.2) (layer "B.Cu") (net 10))
 (segment (start 95.65 76.35) (end 97.38 76.35) (width 0.2) (layer "B.Cu") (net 10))
 (segment (start 95.82 68.73) (end 93 71.55) (width 0.2) (layer "F.Cu") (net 8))
 (segment (start 97.38 68.73) (end 95.82 68.73) (width 0.2) (layer "F.Cu") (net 8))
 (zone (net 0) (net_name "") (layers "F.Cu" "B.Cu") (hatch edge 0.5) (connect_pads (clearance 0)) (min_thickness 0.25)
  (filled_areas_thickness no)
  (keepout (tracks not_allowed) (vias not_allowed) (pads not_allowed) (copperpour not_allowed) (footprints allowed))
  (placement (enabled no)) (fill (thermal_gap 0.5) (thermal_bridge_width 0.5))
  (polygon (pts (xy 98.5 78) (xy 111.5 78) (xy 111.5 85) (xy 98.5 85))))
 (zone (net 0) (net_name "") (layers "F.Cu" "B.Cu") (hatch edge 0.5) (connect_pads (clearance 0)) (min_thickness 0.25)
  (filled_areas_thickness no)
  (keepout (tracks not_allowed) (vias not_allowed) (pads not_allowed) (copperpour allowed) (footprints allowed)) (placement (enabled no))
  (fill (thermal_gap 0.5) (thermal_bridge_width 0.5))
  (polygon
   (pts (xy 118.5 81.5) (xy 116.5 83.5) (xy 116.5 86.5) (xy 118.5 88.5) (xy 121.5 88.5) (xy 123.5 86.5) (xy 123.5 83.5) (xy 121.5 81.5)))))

